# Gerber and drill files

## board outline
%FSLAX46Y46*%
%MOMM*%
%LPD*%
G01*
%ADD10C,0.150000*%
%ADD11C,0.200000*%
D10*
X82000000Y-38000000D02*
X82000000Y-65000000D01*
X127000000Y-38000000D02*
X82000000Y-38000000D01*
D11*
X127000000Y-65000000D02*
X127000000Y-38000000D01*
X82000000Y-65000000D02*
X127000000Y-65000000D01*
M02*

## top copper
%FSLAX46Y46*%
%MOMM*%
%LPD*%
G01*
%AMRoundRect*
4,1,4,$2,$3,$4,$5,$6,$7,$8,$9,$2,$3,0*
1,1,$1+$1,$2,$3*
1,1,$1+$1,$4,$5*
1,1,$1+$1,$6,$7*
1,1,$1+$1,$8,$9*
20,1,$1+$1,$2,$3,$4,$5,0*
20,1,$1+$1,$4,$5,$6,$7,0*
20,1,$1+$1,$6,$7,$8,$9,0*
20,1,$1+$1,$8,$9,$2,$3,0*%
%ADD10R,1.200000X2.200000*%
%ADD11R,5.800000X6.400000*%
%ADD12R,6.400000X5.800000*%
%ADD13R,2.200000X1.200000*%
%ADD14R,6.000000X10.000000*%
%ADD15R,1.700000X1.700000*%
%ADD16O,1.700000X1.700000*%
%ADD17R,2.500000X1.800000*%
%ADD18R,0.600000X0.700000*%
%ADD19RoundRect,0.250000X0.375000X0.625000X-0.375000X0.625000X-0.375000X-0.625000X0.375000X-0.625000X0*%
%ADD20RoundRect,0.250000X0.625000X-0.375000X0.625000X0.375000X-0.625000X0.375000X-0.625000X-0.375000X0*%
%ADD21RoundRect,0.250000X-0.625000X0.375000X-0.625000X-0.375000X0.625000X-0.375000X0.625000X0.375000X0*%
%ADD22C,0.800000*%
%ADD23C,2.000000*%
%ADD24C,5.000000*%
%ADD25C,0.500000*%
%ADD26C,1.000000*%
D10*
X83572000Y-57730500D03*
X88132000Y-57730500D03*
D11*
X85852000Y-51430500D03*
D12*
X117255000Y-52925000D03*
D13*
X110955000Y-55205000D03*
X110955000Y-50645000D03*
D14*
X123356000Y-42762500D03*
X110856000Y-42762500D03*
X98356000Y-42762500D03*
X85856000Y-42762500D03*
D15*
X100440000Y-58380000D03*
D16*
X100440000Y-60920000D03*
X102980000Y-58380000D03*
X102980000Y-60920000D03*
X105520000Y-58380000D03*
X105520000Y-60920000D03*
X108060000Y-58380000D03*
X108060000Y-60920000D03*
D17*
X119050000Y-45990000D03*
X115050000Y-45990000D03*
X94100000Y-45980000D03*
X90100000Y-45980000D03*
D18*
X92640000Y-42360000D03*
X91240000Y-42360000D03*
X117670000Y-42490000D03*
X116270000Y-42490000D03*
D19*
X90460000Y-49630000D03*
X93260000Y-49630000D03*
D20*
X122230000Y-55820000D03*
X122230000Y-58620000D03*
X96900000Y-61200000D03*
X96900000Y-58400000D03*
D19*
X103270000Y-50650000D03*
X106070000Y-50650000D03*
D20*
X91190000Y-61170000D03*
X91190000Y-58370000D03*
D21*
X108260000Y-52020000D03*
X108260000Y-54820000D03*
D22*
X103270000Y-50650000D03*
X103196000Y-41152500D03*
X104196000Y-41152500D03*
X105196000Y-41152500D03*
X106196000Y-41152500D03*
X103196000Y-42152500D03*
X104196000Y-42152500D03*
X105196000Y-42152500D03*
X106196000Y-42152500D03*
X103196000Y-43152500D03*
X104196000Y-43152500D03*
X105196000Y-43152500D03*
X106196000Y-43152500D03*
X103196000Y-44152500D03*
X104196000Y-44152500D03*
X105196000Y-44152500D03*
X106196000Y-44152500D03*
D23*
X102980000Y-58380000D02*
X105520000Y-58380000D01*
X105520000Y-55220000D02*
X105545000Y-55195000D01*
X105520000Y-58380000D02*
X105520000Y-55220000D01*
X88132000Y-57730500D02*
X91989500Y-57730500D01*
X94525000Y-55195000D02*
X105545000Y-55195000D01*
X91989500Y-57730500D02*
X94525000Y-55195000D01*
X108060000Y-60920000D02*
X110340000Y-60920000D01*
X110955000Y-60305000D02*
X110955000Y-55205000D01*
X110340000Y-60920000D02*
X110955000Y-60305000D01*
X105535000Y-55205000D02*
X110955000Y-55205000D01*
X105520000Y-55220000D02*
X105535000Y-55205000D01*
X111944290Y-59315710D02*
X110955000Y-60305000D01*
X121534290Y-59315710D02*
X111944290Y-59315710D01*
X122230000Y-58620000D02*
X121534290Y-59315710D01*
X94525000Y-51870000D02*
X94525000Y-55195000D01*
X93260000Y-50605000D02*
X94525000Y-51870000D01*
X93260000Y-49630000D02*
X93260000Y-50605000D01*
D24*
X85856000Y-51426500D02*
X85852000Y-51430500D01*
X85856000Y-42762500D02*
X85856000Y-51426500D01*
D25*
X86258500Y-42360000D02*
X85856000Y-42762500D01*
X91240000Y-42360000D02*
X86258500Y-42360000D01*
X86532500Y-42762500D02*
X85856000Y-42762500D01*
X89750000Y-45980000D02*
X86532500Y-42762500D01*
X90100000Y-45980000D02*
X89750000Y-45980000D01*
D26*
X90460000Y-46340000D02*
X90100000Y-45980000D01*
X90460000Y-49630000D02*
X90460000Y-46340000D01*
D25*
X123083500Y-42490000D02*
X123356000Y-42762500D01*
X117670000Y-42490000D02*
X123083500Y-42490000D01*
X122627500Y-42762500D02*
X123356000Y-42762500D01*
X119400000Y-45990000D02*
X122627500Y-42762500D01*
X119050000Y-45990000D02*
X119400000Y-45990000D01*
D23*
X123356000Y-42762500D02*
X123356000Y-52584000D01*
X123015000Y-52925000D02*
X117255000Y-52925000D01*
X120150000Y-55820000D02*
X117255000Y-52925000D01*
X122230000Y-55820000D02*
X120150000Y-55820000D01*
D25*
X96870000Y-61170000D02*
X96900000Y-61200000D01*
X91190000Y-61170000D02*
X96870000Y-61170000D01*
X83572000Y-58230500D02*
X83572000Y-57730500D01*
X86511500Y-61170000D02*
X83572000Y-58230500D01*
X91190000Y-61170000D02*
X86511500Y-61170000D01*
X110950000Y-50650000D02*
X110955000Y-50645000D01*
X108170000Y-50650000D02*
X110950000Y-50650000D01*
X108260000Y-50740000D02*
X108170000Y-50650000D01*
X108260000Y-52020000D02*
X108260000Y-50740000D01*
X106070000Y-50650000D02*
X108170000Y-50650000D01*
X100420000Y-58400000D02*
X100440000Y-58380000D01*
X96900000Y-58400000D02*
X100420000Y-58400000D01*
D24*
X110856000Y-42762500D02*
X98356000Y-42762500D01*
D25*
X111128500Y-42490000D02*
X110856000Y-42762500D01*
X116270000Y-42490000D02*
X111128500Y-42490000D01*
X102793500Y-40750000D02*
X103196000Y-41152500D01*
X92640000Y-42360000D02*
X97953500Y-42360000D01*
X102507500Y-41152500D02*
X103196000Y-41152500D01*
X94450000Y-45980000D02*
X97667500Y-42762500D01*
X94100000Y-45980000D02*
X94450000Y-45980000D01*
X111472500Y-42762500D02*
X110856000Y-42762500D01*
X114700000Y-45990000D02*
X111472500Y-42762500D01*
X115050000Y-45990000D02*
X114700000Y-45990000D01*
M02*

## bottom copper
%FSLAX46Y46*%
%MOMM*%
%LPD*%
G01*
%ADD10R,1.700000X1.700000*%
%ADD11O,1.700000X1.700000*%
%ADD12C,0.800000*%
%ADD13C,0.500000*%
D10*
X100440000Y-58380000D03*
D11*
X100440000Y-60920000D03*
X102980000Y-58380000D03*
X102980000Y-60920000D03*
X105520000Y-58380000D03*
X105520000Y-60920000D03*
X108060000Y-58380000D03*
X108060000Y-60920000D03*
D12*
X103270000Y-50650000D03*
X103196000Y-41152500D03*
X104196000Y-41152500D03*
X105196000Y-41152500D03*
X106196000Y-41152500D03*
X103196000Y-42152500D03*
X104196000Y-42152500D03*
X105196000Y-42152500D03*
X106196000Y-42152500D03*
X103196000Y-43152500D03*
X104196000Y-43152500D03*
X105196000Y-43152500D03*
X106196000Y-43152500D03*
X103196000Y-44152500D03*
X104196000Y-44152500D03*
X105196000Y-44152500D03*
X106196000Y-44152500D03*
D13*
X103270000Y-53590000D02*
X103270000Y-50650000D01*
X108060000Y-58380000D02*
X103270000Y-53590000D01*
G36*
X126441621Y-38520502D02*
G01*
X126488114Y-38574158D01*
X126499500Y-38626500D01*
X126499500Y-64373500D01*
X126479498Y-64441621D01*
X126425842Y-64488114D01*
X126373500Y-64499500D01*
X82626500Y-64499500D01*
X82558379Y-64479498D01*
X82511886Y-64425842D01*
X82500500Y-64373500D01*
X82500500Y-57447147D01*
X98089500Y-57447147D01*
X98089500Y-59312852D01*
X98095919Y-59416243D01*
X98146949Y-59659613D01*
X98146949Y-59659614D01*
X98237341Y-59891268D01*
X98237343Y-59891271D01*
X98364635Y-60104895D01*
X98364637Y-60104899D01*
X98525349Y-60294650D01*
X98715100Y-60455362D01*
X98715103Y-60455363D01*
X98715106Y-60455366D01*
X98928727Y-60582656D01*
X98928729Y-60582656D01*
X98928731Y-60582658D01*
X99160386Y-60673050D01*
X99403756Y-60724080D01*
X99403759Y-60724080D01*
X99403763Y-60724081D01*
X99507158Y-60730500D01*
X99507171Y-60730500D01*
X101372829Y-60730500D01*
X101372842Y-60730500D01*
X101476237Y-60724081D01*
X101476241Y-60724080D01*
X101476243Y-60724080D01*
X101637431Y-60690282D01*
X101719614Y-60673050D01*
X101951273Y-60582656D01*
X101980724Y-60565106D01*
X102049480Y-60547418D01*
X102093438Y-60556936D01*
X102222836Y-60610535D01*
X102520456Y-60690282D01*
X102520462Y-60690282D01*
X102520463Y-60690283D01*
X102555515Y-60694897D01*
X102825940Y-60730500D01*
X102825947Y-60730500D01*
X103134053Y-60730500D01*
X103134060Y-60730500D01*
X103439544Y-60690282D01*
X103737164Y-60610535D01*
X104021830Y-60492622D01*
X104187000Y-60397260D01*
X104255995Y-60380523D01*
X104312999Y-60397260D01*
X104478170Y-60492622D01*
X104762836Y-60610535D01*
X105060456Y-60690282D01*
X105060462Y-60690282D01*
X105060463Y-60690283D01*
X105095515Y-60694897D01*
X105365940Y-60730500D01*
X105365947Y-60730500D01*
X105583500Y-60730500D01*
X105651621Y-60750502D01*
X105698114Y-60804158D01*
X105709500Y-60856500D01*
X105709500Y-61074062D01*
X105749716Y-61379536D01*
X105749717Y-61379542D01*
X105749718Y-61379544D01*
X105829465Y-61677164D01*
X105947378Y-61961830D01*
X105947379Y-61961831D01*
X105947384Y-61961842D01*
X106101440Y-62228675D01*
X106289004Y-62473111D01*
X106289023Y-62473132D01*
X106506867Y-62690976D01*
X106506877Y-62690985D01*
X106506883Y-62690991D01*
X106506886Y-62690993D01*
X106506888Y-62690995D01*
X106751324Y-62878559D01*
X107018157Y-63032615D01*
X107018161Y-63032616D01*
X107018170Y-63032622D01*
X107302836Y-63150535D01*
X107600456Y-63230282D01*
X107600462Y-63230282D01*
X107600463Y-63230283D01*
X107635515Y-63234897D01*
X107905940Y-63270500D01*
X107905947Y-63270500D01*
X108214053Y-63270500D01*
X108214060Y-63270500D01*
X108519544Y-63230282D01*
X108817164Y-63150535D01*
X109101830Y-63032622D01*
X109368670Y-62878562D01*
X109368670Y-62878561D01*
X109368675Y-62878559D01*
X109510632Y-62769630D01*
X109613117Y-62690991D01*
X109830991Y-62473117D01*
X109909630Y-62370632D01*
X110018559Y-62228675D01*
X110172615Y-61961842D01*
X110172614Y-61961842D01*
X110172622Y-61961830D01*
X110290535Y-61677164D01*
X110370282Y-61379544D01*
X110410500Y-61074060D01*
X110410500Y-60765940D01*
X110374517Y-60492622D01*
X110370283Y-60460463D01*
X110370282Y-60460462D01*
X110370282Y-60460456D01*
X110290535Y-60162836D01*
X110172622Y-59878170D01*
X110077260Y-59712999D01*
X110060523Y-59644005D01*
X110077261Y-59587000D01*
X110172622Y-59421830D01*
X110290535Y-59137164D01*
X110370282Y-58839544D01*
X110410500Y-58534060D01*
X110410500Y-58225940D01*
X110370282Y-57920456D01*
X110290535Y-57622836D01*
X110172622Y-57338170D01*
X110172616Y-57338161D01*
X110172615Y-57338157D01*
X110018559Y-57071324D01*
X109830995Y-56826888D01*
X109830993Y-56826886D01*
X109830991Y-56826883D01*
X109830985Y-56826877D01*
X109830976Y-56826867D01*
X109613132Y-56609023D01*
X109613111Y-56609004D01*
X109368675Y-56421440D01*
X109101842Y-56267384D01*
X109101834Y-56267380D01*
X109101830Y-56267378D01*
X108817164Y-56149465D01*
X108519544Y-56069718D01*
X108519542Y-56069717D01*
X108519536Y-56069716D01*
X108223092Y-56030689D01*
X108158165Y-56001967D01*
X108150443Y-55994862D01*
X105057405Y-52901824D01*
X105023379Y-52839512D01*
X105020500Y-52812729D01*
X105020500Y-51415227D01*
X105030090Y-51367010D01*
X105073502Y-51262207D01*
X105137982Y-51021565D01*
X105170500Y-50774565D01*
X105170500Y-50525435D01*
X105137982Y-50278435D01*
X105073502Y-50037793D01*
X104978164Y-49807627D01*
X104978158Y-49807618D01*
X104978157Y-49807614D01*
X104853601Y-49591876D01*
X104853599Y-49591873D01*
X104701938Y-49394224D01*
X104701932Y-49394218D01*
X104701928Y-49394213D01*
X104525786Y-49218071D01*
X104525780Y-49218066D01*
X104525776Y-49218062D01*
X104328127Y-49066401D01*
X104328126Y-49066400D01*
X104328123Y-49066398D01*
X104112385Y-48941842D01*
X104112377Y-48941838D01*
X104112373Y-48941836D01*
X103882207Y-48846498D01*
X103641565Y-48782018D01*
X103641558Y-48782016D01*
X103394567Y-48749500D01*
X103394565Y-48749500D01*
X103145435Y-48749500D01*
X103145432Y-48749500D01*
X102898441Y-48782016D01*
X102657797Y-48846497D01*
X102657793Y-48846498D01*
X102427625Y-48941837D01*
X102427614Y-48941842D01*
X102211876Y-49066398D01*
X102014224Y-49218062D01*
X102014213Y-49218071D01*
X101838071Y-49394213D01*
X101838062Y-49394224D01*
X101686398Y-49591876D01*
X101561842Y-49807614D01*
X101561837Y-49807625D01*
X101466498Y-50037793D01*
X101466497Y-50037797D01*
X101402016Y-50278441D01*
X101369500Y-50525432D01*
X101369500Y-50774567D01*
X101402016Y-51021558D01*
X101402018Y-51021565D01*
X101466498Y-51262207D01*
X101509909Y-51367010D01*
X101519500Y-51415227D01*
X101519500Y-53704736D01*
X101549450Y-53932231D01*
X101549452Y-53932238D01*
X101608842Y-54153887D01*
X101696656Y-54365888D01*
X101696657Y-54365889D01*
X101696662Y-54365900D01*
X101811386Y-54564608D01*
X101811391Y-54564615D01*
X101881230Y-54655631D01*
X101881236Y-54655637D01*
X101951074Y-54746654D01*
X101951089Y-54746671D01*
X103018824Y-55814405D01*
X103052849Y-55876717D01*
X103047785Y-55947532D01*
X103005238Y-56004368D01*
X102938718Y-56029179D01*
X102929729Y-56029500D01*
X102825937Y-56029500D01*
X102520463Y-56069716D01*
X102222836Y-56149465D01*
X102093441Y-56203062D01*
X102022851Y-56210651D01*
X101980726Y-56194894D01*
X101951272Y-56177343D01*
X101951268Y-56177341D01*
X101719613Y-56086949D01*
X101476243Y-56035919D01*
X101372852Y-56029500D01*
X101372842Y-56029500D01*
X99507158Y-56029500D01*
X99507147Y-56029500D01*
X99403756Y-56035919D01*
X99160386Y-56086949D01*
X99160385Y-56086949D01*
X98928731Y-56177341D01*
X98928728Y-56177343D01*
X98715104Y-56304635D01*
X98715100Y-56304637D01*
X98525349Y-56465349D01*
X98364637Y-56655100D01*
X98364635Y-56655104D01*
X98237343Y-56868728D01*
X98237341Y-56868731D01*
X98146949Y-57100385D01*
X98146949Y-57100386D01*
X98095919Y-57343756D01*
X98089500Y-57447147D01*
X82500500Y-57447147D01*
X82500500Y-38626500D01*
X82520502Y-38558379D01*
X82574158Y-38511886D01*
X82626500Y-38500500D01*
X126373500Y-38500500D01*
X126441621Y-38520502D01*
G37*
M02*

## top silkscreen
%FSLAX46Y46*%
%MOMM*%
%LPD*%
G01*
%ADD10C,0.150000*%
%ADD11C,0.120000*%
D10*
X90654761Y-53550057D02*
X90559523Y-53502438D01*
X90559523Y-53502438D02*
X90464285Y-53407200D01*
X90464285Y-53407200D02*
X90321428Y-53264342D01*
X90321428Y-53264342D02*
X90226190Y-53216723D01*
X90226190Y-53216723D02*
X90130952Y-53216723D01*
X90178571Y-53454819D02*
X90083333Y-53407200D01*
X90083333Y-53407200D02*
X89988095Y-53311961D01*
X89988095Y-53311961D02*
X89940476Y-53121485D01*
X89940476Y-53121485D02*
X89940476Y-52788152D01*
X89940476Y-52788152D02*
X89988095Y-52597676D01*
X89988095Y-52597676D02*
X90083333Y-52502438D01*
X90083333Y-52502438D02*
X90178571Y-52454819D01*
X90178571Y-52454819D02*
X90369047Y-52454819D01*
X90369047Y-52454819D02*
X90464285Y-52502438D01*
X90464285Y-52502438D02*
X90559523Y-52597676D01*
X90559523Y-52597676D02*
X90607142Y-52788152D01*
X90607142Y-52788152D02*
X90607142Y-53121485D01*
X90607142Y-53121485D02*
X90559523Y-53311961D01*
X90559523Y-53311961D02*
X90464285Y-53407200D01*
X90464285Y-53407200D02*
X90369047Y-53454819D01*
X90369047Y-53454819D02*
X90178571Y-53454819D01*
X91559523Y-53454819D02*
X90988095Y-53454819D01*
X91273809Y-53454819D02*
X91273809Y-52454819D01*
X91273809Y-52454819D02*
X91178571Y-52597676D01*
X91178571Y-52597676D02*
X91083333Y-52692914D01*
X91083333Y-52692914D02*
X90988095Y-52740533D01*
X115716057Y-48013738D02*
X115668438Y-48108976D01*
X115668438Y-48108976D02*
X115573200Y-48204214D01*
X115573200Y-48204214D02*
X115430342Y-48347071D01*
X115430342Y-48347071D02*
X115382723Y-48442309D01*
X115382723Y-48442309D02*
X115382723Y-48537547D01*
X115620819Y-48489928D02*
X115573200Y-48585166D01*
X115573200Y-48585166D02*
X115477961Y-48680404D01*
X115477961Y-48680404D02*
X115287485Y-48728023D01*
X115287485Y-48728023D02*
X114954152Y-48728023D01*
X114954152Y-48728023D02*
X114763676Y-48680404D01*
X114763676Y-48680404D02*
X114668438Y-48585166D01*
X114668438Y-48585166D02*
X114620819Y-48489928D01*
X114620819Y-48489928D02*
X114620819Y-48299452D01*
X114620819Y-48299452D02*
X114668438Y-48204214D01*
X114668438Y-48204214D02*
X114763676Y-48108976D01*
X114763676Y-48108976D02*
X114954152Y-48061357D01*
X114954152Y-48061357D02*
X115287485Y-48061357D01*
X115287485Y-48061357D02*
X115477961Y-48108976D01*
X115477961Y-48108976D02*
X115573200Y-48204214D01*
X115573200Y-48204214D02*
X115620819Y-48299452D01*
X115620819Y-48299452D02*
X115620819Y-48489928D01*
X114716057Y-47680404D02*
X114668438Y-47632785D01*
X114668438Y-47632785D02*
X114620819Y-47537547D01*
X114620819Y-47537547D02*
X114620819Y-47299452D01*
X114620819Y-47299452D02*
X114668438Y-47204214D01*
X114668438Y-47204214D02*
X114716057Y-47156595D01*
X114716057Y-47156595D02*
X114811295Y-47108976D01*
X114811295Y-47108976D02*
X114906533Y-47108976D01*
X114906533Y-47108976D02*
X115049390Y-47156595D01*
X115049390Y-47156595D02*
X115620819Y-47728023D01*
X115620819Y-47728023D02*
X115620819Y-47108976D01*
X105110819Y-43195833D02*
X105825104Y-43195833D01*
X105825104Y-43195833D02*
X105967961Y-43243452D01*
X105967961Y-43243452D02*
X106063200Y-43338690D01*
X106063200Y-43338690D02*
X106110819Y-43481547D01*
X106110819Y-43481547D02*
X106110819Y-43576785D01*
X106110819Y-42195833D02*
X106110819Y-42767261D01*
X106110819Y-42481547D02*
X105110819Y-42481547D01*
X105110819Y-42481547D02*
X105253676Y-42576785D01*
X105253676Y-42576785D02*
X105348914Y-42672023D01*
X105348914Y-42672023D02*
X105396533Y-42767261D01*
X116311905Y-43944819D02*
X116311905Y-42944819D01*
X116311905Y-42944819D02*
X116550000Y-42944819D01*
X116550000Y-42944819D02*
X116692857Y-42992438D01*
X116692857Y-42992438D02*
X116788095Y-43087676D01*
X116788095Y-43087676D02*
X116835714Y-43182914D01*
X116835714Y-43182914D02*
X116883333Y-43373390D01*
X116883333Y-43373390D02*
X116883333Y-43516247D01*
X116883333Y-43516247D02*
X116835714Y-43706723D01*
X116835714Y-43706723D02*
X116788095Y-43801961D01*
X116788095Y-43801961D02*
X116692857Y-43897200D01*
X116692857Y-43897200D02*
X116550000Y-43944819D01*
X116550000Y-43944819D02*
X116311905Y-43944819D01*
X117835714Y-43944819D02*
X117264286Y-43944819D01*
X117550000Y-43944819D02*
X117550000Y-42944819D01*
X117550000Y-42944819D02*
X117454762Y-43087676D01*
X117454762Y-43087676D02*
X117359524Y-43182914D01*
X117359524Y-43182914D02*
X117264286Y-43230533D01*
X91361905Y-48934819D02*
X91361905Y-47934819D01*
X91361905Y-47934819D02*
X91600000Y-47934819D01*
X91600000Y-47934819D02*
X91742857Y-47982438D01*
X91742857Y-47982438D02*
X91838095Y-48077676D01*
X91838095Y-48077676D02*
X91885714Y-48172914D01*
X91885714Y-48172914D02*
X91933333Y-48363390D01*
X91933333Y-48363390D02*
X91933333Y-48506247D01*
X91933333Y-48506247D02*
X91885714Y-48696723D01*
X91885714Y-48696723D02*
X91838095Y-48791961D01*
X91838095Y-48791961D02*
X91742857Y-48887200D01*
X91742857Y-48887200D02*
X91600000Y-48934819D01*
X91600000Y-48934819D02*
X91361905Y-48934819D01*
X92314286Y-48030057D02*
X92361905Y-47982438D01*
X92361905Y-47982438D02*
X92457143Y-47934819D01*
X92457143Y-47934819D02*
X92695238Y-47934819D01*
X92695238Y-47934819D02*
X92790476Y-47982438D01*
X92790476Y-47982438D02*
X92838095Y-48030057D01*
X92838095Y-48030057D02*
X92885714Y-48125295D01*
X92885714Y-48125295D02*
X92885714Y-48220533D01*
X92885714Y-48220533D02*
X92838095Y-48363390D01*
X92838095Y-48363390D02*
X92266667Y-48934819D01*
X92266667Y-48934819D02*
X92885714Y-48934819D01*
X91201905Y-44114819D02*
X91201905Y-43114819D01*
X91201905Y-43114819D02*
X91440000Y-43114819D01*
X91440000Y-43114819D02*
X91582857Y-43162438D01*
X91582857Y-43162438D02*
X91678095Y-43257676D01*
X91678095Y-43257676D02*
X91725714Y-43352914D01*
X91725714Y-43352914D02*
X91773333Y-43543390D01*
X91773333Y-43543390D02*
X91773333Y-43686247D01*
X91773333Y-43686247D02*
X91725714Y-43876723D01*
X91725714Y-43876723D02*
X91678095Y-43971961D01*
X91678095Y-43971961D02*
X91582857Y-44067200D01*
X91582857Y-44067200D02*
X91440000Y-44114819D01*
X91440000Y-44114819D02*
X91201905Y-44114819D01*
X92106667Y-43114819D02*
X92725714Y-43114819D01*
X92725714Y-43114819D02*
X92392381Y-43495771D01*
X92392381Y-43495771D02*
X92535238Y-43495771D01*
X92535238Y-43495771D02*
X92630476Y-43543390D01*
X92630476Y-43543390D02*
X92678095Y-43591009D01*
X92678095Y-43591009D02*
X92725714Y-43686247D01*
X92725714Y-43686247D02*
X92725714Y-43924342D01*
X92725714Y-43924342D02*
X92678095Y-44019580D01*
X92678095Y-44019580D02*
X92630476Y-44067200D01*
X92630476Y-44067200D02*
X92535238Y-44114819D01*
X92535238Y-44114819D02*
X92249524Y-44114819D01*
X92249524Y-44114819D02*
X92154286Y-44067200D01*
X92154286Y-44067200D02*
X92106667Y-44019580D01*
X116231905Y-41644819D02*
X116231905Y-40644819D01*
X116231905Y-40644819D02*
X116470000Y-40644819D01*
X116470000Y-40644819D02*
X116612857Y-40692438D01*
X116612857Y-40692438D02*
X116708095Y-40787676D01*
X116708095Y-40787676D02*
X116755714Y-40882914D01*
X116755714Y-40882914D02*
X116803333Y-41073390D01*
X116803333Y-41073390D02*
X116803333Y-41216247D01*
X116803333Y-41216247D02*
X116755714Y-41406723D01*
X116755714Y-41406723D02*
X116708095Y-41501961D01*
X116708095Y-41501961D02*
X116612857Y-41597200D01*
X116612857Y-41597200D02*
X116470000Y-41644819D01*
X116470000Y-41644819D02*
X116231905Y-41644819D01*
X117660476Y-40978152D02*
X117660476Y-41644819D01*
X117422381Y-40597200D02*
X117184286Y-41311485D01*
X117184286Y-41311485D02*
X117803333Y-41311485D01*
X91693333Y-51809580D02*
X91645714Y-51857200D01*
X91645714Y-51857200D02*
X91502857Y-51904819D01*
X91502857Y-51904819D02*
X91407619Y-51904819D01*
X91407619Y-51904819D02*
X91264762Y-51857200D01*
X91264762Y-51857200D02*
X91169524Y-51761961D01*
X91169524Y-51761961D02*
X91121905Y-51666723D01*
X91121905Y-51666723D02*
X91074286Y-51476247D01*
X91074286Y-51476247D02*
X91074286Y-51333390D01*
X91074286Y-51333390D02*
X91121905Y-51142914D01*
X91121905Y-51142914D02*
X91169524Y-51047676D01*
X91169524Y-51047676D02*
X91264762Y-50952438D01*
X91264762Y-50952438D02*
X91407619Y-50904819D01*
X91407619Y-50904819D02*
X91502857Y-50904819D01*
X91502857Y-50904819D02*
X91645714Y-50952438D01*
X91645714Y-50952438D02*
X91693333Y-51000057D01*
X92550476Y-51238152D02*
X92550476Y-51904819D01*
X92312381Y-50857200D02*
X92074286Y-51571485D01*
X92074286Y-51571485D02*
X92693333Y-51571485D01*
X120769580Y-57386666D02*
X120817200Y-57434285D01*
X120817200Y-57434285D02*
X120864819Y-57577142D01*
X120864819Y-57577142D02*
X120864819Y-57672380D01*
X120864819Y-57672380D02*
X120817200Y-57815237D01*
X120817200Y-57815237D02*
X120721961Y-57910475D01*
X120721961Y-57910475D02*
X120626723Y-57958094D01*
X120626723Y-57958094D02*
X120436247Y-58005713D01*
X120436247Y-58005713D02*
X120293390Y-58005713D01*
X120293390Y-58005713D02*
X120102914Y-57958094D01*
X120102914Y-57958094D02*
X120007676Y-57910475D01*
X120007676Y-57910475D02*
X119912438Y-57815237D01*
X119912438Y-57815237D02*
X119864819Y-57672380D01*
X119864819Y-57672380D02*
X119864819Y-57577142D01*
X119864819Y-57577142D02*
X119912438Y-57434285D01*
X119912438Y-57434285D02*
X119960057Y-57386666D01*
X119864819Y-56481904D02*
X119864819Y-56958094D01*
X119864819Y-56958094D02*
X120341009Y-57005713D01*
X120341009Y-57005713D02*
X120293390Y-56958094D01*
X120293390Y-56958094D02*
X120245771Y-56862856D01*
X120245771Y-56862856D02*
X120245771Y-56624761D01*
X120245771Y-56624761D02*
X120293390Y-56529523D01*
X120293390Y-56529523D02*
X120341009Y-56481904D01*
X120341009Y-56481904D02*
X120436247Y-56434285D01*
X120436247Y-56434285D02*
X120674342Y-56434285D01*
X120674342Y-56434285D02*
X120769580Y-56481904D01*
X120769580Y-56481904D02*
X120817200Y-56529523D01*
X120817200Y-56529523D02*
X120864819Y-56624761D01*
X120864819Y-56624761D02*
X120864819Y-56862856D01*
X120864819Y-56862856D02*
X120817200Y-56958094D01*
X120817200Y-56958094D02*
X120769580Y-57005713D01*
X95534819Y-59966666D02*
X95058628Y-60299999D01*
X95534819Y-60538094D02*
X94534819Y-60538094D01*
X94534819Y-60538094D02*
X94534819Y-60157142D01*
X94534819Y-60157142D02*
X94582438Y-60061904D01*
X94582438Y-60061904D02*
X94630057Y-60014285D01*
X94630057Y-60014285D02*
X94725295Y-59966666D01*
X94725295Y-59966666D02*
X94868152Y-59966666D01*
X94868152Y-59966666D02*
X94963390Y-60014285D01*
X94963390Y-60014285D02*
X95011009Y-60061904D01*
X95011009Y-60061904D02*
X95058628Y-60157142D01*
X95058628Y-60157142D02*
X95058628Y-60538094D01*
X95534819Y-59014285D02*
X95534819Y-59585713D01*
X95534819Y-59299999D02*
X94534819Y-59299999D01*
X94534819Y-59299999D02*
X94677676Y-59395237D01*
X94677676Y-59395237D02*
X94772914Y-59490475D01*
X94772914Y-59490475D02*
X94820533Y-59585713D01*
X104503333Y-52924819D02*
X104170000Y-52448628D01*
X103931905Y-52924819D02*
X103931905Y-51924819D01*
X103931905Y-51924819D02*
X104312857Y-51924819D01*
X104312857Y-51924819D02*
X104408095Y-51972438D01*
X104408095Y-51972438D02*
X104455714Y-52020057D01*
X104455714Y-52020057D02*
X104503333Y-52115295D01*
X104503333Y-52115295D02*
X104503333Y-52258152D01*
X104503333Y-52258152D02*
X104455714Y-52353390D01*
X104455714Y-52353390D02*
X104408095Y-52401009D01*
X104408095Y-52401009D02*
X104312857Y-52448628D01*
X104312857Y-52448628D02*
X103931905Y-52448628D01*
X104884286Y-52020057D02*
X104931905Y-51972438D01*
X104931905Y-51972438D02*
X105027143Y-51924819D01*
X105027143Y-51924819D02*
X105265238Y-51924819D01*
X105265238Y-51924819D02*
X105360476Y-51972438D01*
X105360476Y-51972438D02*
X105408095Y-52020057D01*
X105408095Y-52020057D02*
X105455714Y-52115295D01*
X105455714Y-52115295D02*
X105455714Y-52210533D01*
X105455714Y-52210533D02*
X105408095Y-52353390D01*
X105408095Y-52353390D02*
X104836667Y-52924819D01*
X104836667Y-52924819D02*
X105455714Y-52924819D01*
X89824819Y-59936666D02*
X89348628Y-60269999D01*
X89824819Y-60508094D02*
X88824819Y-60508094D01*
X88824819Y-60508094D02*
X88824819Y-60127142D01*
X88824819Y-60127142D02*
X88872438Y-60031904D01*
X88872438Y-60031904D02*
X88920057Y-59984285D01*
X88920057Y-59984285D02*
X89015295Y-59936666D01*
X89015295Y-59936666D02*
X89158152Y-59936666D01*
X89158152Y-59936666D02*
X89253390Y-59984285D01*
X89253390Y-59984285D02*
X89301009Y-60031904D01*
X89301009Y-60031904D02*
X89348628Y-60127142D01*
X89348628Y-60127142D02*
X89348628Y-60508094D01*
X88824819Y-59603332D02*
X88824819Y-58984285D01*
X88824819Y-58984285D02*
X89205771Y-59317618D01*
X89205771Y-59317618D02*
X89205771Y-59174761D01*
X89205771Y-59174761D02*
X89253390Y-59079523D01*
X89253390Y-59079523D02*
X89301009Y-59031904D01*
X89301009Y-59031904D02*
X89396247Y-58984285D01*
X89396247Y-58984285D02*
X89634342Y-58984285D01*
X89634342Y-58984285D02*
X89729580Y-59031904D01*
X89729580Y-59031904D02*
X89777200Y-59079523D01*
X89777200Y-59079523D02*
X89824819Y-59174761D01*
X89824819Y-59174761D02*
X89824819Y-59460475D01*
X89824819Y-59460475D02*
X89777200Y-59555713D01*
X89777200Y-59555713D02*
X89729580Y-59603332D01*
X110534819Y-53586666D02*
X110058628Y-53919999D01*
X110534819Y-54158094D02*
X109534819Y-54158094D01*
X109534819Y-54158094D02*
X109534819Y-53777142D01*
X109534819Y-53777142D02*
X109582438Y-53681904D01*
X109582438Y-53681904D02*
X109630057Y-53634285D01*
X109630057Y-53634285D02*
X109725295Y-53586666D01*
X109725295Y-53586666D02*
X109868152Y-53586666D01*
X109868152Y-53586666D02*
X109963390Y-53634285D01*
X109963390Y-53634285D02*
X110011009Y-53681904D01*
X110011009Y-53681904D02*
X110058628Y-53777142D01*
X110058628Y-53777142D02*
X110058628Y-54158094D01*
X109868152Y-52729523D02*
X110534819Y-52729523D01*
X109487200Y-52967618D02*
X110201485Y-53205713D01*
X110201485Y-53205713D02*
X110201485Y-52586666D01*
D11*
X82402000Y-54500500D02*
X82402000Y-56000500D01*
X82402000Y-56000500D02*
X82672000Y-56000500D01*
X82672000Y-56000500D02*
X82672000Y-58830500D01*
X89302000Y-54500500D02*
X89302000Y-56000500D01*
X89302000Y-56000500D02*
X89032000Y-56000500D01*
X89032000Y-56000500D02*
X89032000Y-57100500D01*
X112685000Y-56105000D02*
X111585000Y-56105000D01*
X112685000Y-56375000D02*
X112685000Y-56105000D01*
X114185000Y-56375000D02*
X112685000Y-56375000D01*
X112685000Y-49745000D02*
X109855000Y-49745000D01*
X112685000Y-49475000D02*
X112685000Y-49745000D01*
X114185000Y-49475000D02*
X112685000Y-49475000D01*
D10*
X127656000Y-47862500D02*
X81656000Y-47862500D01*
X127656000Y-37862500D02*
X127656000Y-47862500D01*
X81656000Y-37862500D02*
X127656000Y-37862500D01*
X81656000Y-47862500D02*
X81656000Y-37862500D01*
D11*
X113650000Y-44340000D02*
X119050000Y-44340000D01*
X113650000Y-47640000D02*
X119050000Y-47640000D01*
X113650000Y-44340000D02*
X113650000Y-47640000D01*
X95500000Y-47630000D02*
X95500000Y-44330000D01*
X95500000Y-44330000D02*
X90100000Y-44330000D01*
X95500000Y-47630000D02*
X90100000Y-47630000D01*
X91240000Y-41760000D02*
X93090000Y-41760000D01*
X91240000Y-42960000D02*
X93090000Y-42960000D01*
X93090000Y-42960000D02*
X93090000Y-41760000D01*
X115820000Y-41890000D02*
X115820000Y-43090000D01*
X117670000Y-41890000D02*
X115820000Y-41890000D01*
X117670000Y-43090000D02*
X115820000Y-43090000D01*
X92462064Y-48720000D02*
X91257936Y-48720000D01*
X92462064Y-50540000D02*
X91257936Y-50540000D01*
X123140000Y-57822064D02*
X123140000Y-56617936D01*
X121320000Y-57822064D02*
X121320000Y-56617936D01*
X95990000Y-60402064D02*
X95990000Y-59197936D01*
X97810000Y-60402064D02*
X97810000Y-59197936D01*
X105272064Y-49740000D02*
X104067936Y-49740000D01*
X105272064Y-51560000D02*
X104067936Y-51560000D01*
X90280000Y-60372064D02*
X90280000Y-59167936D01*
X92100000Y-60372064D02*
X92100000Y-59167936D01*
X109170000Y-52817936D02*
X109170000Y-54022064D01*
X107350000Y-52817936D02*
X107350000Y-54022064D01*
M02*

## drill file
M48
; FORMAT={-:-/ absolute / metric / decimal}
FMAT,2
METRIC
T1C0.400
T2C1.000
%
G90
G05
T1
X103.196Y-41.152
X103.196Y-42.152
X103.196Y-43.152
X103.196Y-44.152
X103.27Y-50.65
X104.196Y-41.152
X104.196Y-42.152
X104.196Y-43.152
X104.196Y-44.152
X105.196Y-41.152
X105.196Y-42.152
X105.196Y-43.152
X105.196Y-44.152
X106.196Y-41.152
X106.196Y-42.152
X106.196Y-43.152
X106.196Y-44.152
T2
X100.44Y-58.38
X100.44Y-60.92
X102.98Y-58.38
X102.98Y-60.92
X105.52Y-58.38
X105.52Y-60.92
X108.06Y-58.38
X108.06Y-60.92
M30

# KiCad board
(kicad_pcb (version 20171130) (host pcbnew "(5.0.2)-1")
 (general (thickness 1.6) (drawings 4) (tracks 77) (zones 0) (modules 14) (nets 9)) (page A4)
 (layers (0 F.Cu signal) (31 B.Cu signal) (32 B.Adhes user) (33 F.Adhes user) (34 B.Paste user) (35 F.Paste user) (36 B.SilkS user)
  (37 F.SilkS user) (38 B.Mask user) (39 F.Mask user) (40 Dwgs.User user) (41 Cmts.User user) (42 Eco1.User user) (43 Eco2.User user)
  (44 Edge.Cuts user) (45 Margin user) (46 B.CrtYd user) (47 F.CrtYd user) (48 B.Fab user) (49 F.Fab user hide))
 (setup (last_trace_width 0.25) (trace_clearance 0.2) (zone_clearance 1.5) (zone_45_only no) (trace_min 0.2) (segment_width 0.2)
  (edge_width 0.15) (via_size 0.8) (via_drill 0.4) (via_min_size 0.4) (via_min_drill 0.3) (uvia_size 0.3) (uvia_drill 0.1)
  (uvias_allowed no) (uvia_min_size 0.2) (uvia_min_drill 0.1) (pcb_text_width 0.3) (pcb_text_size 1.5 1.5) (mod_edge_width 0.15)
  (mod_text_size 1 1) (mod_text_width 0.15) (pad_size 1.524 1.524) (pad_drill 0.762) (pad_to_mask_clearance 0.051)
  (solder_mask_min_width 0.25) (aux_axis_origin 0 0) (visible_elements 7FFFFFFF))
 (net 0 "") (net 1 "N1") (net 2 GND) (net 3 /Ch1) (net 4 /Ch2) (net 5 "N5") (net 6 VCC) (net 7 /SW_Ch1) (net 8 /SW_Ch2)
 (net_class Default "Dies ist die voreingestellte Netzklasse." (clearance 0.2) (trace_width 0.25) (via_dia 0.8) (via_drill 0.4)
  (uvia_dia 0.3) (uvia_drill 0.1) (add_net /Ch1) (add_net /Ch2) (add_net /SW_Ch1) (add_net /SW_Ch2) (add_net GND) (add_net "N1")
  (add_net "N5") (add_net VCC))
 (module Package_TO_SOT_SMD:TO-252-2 (layer F.Cu) (at 85.852 53.5305 90)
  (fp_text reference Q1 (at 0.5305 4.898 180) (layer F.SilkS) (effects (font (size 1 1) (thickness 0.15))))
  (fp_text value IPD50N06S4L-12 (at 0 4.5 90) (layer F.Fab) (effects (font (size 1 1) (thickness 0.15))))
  (fp_line (start -0.97 -3.45) (end -2.47 -3.45) (layer F.SilkS) (width 0.12))
  (fp_line (start -2.47 -3.45) (end -2.47 -3.18) (layer F.SilkS) (width 0.12))
  (fp_line (start -2.47 -3.18) (end -5.3 -3.18) (layer F.SilkS) (width 0.12))
  (fp_line (start -0.97 3.45) (end -2.47 3.45) (layer F.SilkS) (width 0.12))
  (fp_line (start -2.47 3.45) (end -2.47 3.18) (layer F.SilkS) (width 0.12))
  (fp_line (start -2.47 3.18) (end -3.57 3.18) (layer F.SilkS) (width 0.12))
  (pad 1 smd rect (at -4.2 -2.28 90) (size 2.2 1.2) (layers F.Cu F.Paste F.Mask) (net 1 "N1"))
  (pad 3 smd rect (at -4.2 2.28 90) (size 2.2 1.2) (layers F.Cu F.Paste F.Mask) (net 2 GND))
  (pad 2 smd rect (at 2.1 0 90) (size 6.4 5.8) (layers F.Cu F.Mask) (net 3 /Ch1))
  (pad "" smd rect (at 3.775 1.525 90) (size 3.05 2.75) (layers F.Paste))
  (pad "" smd rect (at 0.425 -1.525 90) (size 3.05 2.75) (layers F.Paste))
  (pad "" smd rect (at 3.775 -1.525 90) (size 3.05 2.75) (layers F.Paste))
  (pad "" smd rect (at 0.425 1.525 90) (size 3.05 2.75) (layers F.Paste)))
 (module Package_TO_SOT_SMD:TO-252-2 (layer F.Cu) (at 115.155 52.925)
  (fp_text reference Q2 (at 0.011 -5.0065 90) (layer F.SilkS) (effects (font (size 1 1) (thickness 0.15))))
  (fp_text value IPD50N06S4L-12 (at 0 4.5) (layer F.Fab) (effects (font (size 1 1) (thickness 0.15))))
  (fp_line (start -2.47 3.18) (end -3.57 3.18) (layer F.SilkS) (width 0.12))
  (fp_line (start -2.47 3.45) (end -2.47 3.18) (layer F.SilkS) (width 0.12))
  (fp_line (start -0.97 3.45) (end -2.47 3.45) (layer F.SilkS) (width 0.12))
  (fp_line (start -2.47 -3.18) (end -5.3 -3.18) (layer F.SilkS) (width 0.12))
  (fp_line (start -2.47 -3.45) (end -2.47 -3.18) (layer F.SilkS) (width 0.12))
  (fp_line (start -0.97 -3.45) (end -2.47 -3.45) (layer F.SilkS) (width 0.12))
  (pad "" smd rect (at 0.425 1.525) (size 3.05 2.75) (layers F.Paste))
  (pad "" smd rect (at 3.775 -1.525) (size 3.05 2.75) (layers F.Paste))
  (pad "" smd rect (at 0.425 -1.525) (size 3.05 2.75) (layers F.Paste))
  (pad "" smd rect (at 3.775 1.525) (size 3.05 2.75) (layers F.Paste))
  (pad 2 smd rect (at 2.1 0) (size 6.4 5.8) (layers F.Cu F.Mask) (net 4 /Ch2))
  (pad 3 smd rect (at -4.2 2.28) (size 2.2 1.2) (layers F.Cu F.Paste F.Mask) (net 2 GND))
  (pad 1 smd rect (at -4.2 -2.28) (size 2.2 1.2) (layers F.Cu F.Paste F.Mask) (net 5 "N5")))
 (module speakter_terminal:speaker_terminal (layer F.Cu) (at 105.156 42.8625 90)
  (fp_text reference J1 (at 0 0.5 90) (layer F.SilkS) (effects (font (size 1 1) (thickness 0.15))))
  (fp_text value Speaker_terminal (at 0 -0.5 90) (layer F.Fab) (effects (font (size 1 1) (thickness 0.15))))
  (fp_line (start -5 22.5) (end -5 -23.5) (layer F.SilkS) (width 0.15))
  (fp_line (start 5 22.5) (end -5 22.5) (layer F.SilkS) (width 0.15))
  (fp_line (start 5 -23.5) (end 5 22.5) (layer F.SilkS) (width 0.15))
  (fp_line (start -5 -23.5) (end 5 -23.5) (layer F.SilkS) (width 0.15))
  (pad 4 smd rect (at 0.1 18.2 90) (size 10 6) (layers F.Cu F.Paste F.Mask) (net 4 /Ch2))
  (pad 3 smd rect (at 0.1 5.7 90) (size 10 6) (layers F.Cu F.Paste F.Mask) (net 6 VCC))
  (pad 2 smd rect (at 0.1 -6.8 90) (size 10 6) (layers F.Cu F.Paste F.Mask) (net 6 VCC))
  (pad 1 smd rect (at 0.1 -19.3 90) (size 10 6) (layers F.Cu F.Paste F.Mask) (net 3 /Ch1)))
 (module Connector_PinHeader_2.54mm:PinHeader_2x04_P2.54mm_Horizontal (layer B.Cu) (at 100.44 58.38 270)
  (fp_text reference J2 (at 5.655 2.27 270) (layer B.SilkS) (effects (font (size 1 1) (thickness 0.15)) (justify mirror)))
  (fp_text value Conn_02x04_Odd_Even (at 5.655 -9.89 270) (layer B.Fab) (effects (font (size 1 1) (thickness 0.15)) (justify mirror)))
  (pad 1 thru_hole rect (at 0 0 270) (size 1.7 1.7) (drill 1) (layers *.Cu *.Mask) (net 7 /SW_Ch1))
  (pad 2 thru_hole oval (at 2.54 0 270) (size 1.7 1.7) (drill 1) (layers *.Cu *.Mask) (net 6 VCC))
  (pad 3 thru_hole oval (at 0 -2.54 270) (size 1.7 1.7) (drill 1) (layers *.Cu *.Mask) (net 2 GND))
  (pad 4 thru_hole oval (at 2.54 -2.54 270) (size 1.7 1.7) (drill 1) (layers *.Cu *.Mask) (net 6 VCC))
  (pad 5 thru_hole oval (at 0 -5.08 270) (size 1.7 1.7) (drill 1) (layers *.Cu *.Mask) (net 2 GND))
  (pad 6 thru_hole oval (at 2.54 -5.08 270) (size 1.7 1.7) (drill 1) (layers *.Cu *.Mask) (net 6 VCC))
  (pad 7 thru_hole oval (at 0 -7.62 270) (size 1.7 1.7) (drill 1) (layers *.Cu *.Mask) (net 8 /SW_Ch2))
  (pad 8 thru_hole oval (at 2.54 -7.62 270) (size 1.7 1.7) (drill 1) (layers *.Cu *.Mask) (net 2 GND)))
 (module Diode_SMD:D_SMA (layer F.Cu) (at 117.05 45.99)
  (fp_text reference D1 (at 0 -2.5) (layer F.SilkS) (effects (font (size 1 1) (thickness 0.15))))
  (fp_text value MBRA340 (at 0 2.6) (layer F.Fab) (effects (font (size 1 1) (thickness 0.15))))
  (fp_line (start -3.4 -1.65) (end 2 -1.65) (layer F.SilkS) (width 0.12))
  (fp_line (start -3.4 1.65) (end 2 1.65) (layer F.SilkS) (width 0.12))
  (fp_line (start -3.4 -1.65) (end -3.4 1.65) (layer F.SilkS) (width 0.12))
  (pad 2 smd rect (at 2 0) (size 2.5 1.8) (layers F.Cu F.Paste F.Mask) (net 4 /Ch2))
  (pad 1 smd rect (at -2 0) (size 2.5 1.8) (layers F.Cu F.Paste F.Mask) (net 6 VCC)))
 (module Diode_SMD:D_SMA (layer F.Cu) (at 92.1 45.98 180)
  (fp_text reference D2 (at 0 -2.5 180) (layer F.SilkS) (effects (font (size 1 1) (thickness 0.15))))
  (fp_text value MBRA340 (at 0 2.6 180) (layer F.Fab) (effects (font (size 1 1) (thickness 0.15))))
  (fp_line (start -3.4 -1.65) (end -3.4 1.65) (layer F.SilkS) (width 0.12))
  (fp_line (start -3.4 1.65) (end 2 1.65) (layer F.SilkS) (width 0.12))
  (fp_line (start -3.4 -1.65) (end 2 -1.65) (layer F.SilkS) (width 0.12))
  (pad 1 smd rect (at -2 0 180) (size 2.5 1.8) (layers F.Cu F.Paste F.Mask) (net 6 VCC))
  (pad 2 smd rect (at 2 0 180) (size 2.5 1.8) (layers F.Cu F.Paste F.Mask) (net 3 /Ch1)))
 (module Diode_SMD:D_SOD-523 (layer F.Cu) (at 91.94 42.36 180)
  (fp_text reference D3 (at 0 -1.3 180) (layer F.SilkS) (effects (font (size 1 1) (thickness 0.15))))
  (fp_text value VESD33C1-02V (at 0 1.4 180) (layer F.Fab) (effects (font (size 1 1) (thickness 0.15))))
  (fp_line (start 0.7 0.6) (end -1.15 0.6) (layer F.SilkS) (width 0.12))
  (fp_line (start 0.7 -0.6) (end -1.15 -0.6) (layer F.SilkS) (width 0.12))
  (fp_line (start -1.15 -0.6) (end -1.15 0.6) (layer F.SilkS) (width 0.12))
  (pad 1 smd rect (at -0.7 0) (size 0.6 0.7) (layers F.Cu F.Paste F.Mask) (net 6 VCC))
  (pad 2 smd rect (at 0.7 0) (size 0.6 0.7) (layers F.Cu F.Paste F.Mask) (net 3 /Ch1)))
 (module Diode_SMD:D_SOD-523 (layer F.Cu) (at 116.97 42.49)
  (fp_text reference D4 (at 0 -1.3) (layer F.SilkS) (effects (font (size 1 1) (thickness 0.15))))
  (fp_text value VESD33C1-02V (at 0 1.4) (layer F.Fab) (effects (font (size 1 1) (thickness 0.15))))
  (fp_line (start -1.15 -0.6) (end -1.15 0.6) (layer F.SilkS) (width 0.12))
  (fp_line (start 0.7 -0.6) (end -1.15 -0.6) (layer F.SilkS) (width 0.12))
  (fp_line (start 0.7 0.6) (end -1.15 0.6) (layer F.SilkS) (width 0.12))
  (pad 2 smd rect (at 0.7 0 180) (size 0.6 0.7) (layers F.Cu F.Paste F.Mask) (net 4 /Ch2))
  (pad 1 smd rect (at -0.7 0 180) (size 0.6 0.7) (layers F.Cu F.Paste F.Mask) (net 6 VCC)))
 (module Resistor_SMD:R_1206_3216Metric (layer F.Cu) (at 91.86 49.63 180)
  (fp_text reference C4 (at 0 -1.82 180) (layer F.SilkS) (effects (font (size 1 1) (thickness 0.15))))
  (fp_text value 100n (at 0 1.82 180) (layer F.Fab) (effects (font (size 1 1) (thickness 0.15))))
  (fp_line (start -0.602064 0.91) (end 0.602064 0.91) (layer F.SilkS) (width 0.12))
  (fp_line (start -0.602064 -0.91) (end 0.602064 -0.91) (layer F.SilkS) (width 0.12))
  (pad 2 smd roundrect (at 1.4 0 180) (size 1.25 1.75) (layers F.Cu F.Paste F.Mask) (roundrect_rratio 0.2) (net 3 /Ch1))
  (pad 1 smd roundrect (at -1.4 0 180) (size 1.25 1.75) (layers F.Cu F.Paste F.Mask) (roundrect_rratio 0.2) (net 2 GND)))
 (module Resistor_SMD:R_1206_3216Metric (layer F.Cu) (at 122.23 57.22 90)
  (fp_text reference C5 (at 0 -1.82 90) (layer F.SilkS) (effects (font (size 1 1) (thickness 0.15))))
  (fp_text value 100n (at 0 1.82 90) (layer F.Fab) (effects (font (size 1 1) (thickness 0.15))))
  (fp_line (start -0.602064 0.91) (end 0.602064 0.91) (layer F.SilkS) (width 0.12))
  (fp_line (start -0.602064 -0.91) (end 0.602064 -0.91) (layer F.SilkS) (width 0.12))
  (pad 2 smd roundrect (at 1.4 0 90) (size 1.25 1.75) (layers F.Cu F.Paste F.Mask) (roundrect_rratio 0.2) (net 4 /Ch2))
  (pad 1 smd roundrect (at -1.4 0 90) (size 1.25 1.75) (layers F.Cu F.Paste F.Mask) (roundrect_rratio 0.2) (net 2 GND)))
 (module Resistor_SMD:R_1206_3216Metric (layer F.Cu) (at 96.9 59.8 90)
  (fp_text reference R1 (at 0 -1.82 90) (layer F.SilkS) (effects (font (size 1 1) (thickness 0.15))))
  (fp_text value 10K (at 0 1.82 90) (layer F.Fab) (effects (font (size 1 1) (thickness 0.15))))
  (fp_line (start -0.602064 -0.91) (end 0.602064 -0.91) (layer F.SilkS) (width 0.12))
  (fp_line (start -0.602064 0.91) (end 0.602064 0.91) (layer F.SilkS) (width 0.12))
  (pad 1 smd roundrect (at -1.4 0 90) (size 1.25 1.75) (layers F.Cu F.Paste F.Mask) (roundrect_rratio 0.2) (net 1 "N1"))
  (pad 2 smd roundrect (at 1.4 0 90) (size 1.25 1.75) (layers F.Cu F.Paste F.Mask) (roundrect_rratio 0.2) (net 7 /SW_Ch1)))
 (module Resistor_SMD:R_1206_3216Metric (layer F.Cu) (at 104.67 50.65 180)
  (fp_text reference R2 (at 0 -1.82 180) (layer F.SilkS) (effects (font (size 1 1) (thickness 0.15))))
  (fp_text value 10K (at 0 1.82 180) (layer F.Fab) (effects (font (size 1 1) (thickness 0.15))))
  (fp_line (start -0.602064 0.91) (end 0.602064 0.91) (layer F.SilkS) (width 0.12))
  (fp_line (start -0.602064 -0.91) (end 0.602064 -0.91) (layer F.SilkS) (width 0.12))
  (pad 2 smd roundrect (at 1.4 0 180) (size 1.25 1.75) (layers F.Cu F.Paste F.Mask) (roundrect_rratio 0.2) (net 8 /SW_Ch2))
  (pad 1 smd roundrect (at -1.4 0 180) (size 1.25 1.75) (layers F.Cu F.Paste F.Mask) (roundrect_rratio 0.2) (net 5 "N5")))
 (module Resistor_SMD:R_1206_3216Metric (layer F.Cu) (at 91.19 59.77 90)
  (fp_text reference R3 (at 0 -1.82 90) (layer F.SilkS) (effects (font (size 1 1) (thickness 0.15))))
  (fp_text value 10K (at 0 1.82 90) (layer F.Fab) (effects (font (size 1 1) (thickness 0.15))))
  (fp_line (start -0.602064 -0.91) (end 0.602064 -0.91) (layer F.SilkS) (width 0.12))
  (fp_line (start -0.602064 0.91) (end 0.602064 0.91) (layer F.SilkS) (width 0.12))
  (pad 1 smd roundrect (at -1.4 0 90) (size 1.25 1.75) (layers F.Cu F.Paste F.Mask) (roundrect_rratio 0.2) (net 1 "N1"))
  (pad 2 smd roundrect (at 1.4 0 90) (size 1.25 1.75) (layers F.Cu F.Paste F.Mask) (roundrect_rratio 0.2) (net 2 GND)))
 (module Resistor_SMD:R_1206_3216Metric (layer F.Cu) (at 108.26 53.42 270)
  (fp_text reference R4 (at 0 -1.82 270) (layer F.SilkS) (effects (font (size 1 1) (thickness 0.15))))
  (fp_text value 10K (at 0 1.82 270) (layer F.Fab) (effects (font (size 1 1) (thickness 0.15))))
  (fp_line (start -0.602064 -0.91) (end 0.602064 -0.91) (layer F.SilkS) (width 0.12))
  (fp_line (start -0.602064 0.91) (end 0.602064 0.91) (layer F.SilkS) (width 0.12))
  (pad 1 smd roundrect (at -1.4 0 270) (size 1.25 1.75) (layers F.Cu F.Paste F.Mask) (roundrect_rratio 0.2) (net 5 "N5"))
  (pad 2 smd roundrect (at 1.4 0 270) (size 1.25 1.75) (layers F.Cu F.Paste F.Mask) (roundrect_rratio 0.2) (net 2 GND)))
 (gr_line (start 82 38) (end 82 65) (layer Edge.Cuts) (width 0.15))
 (gr_line (start 127 38) (end 82 38) (layer Edge.Cuts) (width 0.15))
 (gr_line (start 127 65) (end 127 38) (layer Edge.Cuts) (width 0.2))
 (gr_line (start 82 65) (end 127 65) (layer Edge.Cuts) (width 0.2))
 (segment (start 102.98 58.38) (end 105.52 58.38) (width 2) (layer F.Cu) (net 2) (status 30))
 (segment (start 105.52 55.22) (end 105.545 55.195) (width 2) (layer F.Cu) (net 2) (status 30))
 (segment (start 105.52 58.38) (end 105.52 55.22) (width 2) (layer F.Cu) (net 2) (status 30))
 (segment (start 88.132 57.7305) (end 91.9895 57.7305) (width 2) (layer F.Cu) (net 2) (status 10))
 (segment (start 94.525 55.195) (end 105.545 55.195) (width 2) (layer F.Cu) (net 2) (status 20))
 (segment (start 91.9895 57.7305) (end 94.525 55.195) (width 2) (layer F.Cu) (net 2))
 (segment (start 108.06 60.92) (end 110.34 60.92) (width 2) (layer F.Cu) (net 2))
 (segment (start 110.955 60.305) (end 110.955 55.205) (width 2) (layer F.Cu) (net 2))
 (segment (start 110.34 60.92) (end 110.955 60.305) (width 2) (layer F.Cu) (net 2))
 (segment (start 105.535 55.205) (end 110.955 55.205) (width 2) (layer F.Cu) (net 2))
 (segment (start 105.52 55.22) (end 105.535 55.205) (width 2) (layer F.Cu) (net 2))
 (segment (start 111.94429 59.31571) (end 110.955 60.305) (width 2) (layer F.Cu) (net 2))
 (segment (start 121.53429 59.31571) (end 111.94429 59.31571) (width 2) (layer F.Cu) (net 2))
 (segment (start 122.23 58.62) (end 121.53429 59.31571) (width 2) (layer F.Cu) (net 2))
 (segment (start 94.525 51.87) (end 94.525 55.195) (width 2) (layer F.Cu) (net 2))
 (segment (start 93.26 50.605) (end 94.525 51.87) (width 2) (layer F.Cu) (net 2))
 (segment (start 93.26 49.63) (end 93.26 50.605) (width 2) (layer F.Cu) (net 2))
 (segment (start 85.856 51.4265) (end 85.852 51.4305) (width 5) (layer F.Cu) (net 3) (status 30))
 (segment (start 85.856 42.7625) (end 85.856 51.4265) (width 5) (layer F.Cu) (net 3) (status 30))
 (segment (start 86.2585 42.36) (end 85.856 42.7625) (width 0.5) (layer F.Cu) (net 3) (status 30))
 (segment (start 91.24 42.36) (end 86.2585 42.36) (width 0.5) (layer F.Cu) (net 3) (status 30))
 (segment (start 86.5325 42.7625) (end 85.856 42.7625) (width 0.5) (layer F.Cu) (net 3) (status 30))
 (segment (start 89.75 45.98) (end 86.5325 42.7625) (width 0.5) (layer F.Cu) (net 3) (status 30))
 (segment (start 90.1 45.98) (end 89.75 45.98) (width 0.5) (layer F.Cu) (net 3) (status 30))
 (segment (start 90.46 46.34) (end 90.1 45.98) (width 1) (layer F.Cu) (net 3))
 (segment (start 90.46 49.63) (end 90.46 46.34) (width 1) (layer F.Cu) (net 3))
 (segment (start 123.0835 42.49) (end 123.356 42.7625) (width 0.5) (layer F.Cu) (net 4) (status 30))
 (segment (start 117.67 42.49) (end 123.0835 42.49) (width 0.5) (layer F.Cu) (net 4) (status 30))
 (segment (start 122.6275 42.7625) (end 123.356 42.7625) (width 0.5) (layer F.Cu) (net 4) (status 30))
 (segment (start 119.4 45.99) (end 122.6275 42.7625) (width 0.5) (layer F.Cu) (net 4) (status 30))
 (segment (start 119.05 45.99) (end 119.4 45.99) (width 0.5) (layer F.Cu) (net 4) (status 30))
 (segment (start 123.356 42.7625) (end 123.356 52.584) (width 2) (layer F.Cu) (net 4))
 (segment (start 123.015 52.925) (end 117.255 52.925) (width 2) (layer F.Cu) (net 4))
 (segment (start 120.15 55.82) (end 117.255 52.925) (width 2) (layer F.Cu) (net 4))
 (segment (start 122.23 55.82) (end 120.15 55.82) (width 2) (layer F.Cu) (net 4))
 (segment (start 96.87 61.17) (end 96.9 61.2) (width 0.5) (layer F.Cu) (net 1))
 (segment (start 91.19 61.17) (end 96.87 61.17) (width 0.5) (layer F.Cu) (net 1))
 (segment (start 83.572 58.2305) (end 83.572 57.7305) (width 0.5) (layer F.Cu) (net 1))
 (segment (start 86.5115 61.17) (end 83.572 58.2305) (width 0.5) (layer F.Cu) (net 1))
 (segment (start 91.19 61.17) (end 86.5115 61.17) (width 0.5) (layer F.Cu) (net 1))
 (segment (start 110.95 50.65) (end 110.955 50.645) (width 0.5) (layer F.Cu) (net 5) (status 1000000))
 (segment (start 108.17 50.65) (end 110.95 50.65) (width 0.5) (layer F.Cu) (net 5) (status 1000000))
 (segment (start 108.26 50.74) (end 108.17 50.65) (width 0.5) (layer F.Cu) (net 5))
 (segment (start 108.26 52.02) (end 108.26 50.74) (width 0.5) (layer F.Cu) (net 5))
 (segment (start 106.07 50.65) (end 108.17 50.65) (width 0.5) (layer F.Cu) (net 5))
 (segment (start 100.42 58.4) (end 100.44 58.38) (width 0.5) (layer F.Cu) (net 7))
 (segment (start 96.9 58.4) (end 100.42 58.4) (width 0.5) (layer F.Cu) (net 7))
 (via (at 103.27 50.65) (size 0.8) (drill 0.4) (layers F.Cu B.Cu) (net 8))
 (segment (start 103.27 53.59) (end 103.27 50.65) (width 0.5) (layer B.Cu) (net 8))
 (segment (start 108.06 58.38) (end 103.27 53.59) (width 0.5) (layer B.Cu) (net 8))
 (segment (start 110.856 42.7625) (end 98.356 42.7625) (width 5) (layer F.Cu) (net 6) (status 30))
 (segment (start 111.1285 42.49) (end 110.856 42.7625) (width 0.5) (layer F.Cu) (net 6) (status 30))
 (segment (start 116.27 42.49) (end 111.1285 42.49) (width 0.5) (layer F.Cu) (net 6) (status 30))
 (segment (start 102.7935 40.75) (end 103.196 41.1525) (width 0.5) (layer F.Cu) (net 6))
 (segment (start 92.64 42.36) (end 97.9535 42.36) (width 0.5) (layer F.Cu) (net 6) (status 30))
 (segment (start 102.5075 41.1525) (end 103.196 41.1525) (width 0.5) (layer F.Cu) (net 6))
 (segment (start 94.45 45.98) (end 97.6675 42.7625) (width 0.5) (layer F.Cu) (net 6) (status 30))
 (segment (start 94.1 45.98) (end 94.45 45.98) (width 0.5) (layer F.Cu) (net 6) (status 30))
 (segment (start 111.4725 42.7625) (end 110.856 42.7625) (width 0.5) (layer F.Cu) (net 6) (status 30))
 (segment (start 114.7 45.99) (end 111.4725 42.7625) (width 0.5) (layer F.Cu) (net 6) (status 30))
 (segment (start 115.05 45.99) (end 114.7 45.99) (width 0.5) (layer F.Cu) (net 6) (status 30))
 (via (at 103.196 41.1525) (size 0.8) (drill 0.4) (layers F.Cu B.Cu) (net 6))
 (via (at 104.196 41.1525) (size 0.8) (drill 0.4) (layers F.Cu B.Cu) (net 6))
 (via (at 105.196 41.1525) (size 0.8) (drill 0.4) (layers F.Cu B.Cu) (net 6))
 (via (at 106.196 41.1525) (size 0.8) (drill 0.4) (layers F.Cu B.Cu) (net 6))
 (via (at 103.196 42.1525) (size 0.8) (drill 0.4) (layers F.Cu B.Cu) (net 6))
 (via (at 104.196 42.1525) (size 0.8) (drill 0.4) (layers F.Cu B.Cu) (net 6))
 (via (at 105.196 42.1525) (size 0.8) (drill 0.4) (layers F.Cu B.Cu) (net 6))
 (via (at 106.196 42.1525) (size 0.8) (drill 0.4) (layers F.Cu B.Cu) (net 6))
 (via (at 103.196 43.1525) (size 0.8) (drill 0.4) (layers F.Cu B.Cu) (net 6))
 (via (at 104.196 43.1525) (size 0.8) (drill 0.4) (layers F.Cu B.Cu) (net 6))
 (via (at 105.196 43.1525) (size 0.8) (drill 0.4) (layers F.Cu B.Cu) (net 6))
 (via (at 106.196 43.1525) (size 0.8) (drill 0.4) (layers F.Cu B.Cu) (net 6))
 (via (at 103.196 44.1525) (size 0.8) (drill 0.4) (layers F.Cu B.Cu) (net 6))
 (via (at 104.196 44.1525) (size 0.8) (drill 0.4) (layers F.Cu B.Cu) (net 6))
 (via (at 105.196 44.1525) (size 0.8) (drill 0.4) (layers F.Cu B.Cu) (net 6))
 (via (at 106.196 44.1525) (size 0.8) (drill 0.4) (layers F.Cu B.Cu) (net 6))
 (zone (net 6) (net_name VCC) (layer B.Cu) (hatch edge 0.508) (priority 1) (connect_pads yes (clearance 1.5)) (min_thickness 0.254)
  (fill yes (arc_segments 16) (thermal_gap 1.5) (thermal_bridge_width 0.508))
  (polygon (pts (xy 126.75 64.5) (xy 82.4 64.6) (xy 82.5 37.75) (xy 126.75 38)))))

